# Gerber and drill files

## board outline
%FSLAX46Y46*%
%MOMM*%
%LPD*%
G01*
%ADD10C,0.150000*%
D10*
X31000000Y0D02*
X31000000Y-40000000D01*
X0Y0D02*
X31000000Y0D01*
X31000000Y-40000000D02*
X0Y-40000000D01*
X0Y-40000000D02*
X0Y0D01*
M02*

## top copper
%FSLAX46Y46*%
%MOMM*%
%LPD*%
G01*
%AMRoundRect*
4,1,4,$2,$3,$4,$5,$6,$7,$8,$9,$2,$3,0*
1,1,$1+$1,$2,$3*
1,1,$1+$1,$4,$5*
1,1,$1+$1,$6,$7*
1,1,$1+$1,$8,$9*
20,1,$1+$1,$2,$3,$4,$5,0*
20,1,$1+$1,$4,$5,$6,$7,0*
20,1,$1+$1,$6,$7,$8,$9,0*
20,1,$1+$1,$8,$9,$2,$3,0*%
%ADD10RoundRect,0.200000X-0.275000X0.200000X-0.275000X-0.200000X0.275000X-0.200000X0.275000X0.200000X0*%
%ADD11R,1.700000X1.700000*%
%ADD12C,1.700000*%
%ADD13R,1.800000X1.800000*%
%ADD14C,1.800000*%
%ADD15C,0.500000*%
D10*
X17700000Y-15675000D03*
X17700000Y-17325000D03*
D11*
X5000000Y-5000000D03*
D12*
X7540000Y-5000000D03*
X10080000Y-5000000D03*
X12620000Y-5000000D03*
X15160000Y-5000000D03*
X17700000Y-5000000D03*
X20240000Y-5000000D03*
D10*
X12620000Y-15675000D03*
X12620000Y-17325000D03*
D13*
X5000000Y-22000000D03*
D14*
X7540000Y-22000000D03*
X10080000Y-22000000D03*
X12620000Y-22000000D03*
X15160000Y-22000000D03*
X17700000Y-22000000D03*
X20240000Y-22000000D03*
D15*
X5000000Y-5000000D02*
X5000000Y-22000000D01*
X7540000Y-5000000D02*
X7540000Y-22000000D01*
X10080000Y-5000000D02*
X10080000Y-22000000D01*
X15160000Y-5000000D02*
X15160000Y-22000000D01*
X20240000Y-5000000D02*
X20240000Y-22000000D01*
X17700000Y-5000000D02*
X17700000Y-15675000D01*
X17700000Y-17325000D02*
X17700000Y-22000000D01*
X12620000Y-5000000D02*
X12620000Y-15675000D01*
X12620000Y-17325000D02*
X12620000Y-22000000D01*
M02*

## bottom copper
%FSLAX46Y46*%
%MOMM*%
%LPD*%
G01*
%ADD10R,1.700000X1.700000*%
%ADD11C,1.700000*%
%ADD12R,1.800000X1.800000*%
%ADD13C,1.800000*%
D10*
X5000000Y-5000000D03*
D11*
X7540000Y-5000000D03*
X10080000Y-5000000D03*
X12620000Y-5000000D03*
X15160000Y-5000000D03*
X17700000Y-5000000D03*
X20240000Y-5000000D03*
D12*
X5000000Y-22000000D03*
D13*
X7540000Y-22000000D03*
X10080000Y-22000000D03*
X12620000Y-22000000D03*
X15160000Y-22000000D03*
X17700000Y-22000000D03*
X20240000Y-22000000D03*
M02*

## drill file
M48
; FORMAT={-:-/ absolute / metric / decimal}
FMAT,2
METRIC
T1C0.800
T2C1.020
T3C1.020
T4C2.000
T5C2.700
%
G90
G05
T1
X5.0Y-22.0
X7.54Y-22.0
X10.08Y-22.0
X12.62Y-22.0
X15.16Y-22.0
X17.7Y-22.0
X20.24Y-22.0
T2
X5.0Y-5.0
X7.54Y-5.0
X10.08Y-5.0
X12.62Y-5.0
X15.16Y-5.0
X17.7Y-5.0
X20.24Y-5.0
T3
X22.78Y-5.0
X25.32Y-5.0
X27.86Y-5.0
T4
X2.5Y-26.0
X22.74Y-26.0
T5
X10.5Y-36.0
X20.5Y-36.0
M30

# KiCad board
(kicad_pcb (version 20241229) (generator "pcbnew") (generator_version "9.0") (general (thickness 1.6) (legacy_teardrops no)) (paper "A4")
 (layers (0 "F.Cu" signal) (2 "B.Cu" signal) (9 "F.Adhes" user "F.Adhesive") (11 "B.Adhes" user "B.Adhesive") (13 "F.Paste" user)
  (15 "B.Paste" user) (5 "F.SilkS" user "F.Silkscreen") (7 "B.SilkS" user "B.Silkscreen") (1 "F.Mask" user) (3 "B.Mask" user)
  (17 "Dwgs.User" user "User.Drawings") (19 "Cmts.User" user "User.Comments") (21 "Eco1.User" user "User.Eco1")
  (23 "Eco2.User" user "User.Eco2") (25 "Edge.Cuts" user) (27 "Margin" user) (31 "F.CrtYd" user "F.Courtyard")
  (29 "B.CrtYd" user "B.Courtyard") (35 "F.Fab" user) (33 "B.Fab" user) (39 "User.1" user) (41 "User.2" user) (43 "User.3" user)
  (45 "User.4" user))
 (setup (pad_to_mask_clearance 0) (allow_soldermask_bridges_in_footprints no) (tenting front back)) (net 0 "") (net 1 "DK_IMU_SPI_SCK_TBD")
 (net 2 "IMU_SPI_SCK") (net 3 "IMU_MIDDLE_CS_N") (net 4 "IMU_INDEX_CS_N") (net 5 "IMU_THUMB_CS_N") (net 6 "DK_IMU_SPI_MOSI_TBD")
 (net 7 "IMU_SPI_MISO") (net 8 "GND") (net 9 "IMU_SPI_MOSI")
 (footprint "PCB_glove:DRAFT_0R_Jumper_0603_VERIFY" (layer "F.Cu") (at 17.7 16.5 -90)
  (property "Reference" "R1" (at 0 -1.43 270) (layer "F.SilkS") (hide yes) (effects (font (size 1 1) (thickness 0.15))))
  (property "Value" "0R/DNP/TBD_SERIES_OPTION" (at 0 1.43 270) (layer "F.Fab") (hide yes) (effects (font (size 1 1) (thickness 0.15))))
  (pad "1" smd roundrect (at -0.825 0 270) (size 0.8 0.95) (layers "F.Cu" "F.Mask" "F.Paste") (roundrect_rratio 0.25)
   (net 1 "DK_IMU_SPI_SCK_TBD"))
  (pad "2" smd roundrect (at 0.825 0 270) (size 0.8 0.95) (layers "F.Cu" "F.Mask" "F.Paste") (roundrect_rratio 0.25) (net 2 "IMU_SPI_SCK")))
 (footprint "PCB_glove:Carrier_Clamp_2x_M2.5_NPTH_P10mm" (layer "F.Cu") (at 15.5 36)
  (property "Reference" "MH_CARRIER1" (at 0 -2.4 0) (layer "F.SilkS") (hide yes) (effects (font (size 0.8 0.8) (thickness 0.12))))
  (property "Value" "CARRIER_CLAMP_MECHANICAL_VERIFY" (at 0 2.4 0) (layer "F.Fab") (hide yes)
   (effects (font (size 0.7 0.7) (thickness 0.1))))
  (pad "" np_thru_hole circle (at -5 0) (size 2.7 2.7) (drill 2.7) (layers "*.Cu" "*.Mask"))
  (pad "" np_thru_hole circle (at 5 0) (size 2.7 2.7) (drill 2.7) (layers "*.Cu" "*.Mask")))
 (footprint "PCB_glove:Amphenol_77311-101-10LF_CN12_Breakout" (layer "F.Cu") (at 5 5)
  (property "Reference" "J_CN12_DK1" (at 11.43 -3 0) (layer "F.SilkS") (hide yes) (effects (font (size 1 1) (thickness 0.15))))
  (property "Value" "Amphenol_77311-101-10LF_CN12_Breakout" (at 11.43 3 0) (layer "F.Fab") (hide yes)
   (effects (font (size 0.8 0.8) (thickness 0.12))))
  (pad "" np_thru_hole circle (at 17.78 0) (size 1.02 1.02) (drill 1.02) (layers "*.Cu" "*.Mask"))
  (pad "" np_thru_hole circle (at 20.32 0) (size 1.02 1.02) (drill 1.02) (layers "*.Cu" "*.Mask"))
  (pad "" np_thru_hole circle (at 22.86 0) (size 1.02 1.02) (drill 1.02) (layers "*.Cu" "*.Mask"))
  (pad "1" thru_hole rect (at 0 0) (size 1.7 1.7) (drill 1.02) (layers "*.Cu" "*.Mask") (remove_unused_layers no) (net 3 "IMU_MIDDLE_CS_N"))
  (pad "2" thru_hole circle (at 2.54 0) (size 1.7 1.7) (drill 1.02) (layers "*.Cu" "*.Mask") (remove_unused_layers no)
   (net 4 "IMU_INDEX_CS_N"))
  (pad "3" thru_hole circle (at 5.08 0) (size 1.7 1.7) (drill 1.02) (layers "*.Cu" "*.Mask") (remove_unused_layers no)
   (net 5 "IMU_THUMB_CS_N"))
  (pad "4" thru_hole circle (at 7.62 0) (size 1.7 1.7) (drill 1.02) (layers "*.Cu" "*.Mask") (remove_unused_layers no)
   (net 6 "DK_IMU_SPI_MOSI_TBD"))
  (pad "5" thru_hole circle (at 10.16 0) (size 1.7 1.7) (drill 1.02) (layers "*.Cu" "*.Mask") (remove_unused_layers no)
   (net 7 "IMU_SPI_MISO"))
  (pad "6" thru_hole circle (at 12.7 0) (size 1.7 1.7) (drill 1.02) (layers "*.Cu" "*.Mask") (remove_unused_layers no)
   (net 1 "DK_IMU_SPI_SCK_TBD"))
  (pad "7" thru_hole circle (at 15.24 0) (size 1.7 1.7) (drill 1.02) (layers "*.Cu" "*.Mask") (remove_unused_layers no) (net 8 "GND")))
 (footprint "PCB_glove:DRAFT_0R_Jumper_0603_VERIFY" (layer "F.Cu") (at 12.62 16.5 -90)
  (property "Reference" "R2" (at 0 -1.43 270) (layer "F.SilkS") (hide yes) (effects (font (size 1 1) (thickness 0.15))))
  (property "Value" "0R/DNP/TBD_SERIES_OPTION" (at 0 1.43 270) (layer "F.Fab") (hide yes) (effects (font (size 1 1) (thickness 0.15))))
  (pad "1" smd roundrect (at -0.825 0 270) (size 0.8 0.95) (layers "F.Cu" "F.Mask" "F.Paste") (roundrect_rratio 0.25)
   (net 6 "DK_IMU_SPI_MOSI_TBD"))
  (pad "2" smd roundrect (at 0.825 0 270) (size 0.8 0.95) (layers "F.Cu" "F.Mask" "F.Paste") (roundrect_rratio 0.25) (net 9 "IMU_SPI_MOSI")))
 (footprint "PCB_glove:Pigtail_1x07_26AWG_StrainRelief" (layer "F.Cu") (at 5 22)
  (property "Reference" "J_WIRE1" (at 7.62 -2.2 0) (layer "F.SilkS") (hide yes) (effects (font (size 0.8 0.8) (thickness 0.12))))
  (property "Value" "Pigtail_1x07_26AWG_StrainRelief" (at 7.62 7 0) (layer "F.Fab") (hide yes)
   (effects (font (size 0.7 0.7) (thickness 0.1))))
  (pad "" np_thru_hole circle (at -2.5 4) (size 2 2) (drill 2) (layers "*.Cu" "*.Mask"))
  (pad "" np_thru_hole circle (at 17.74 4) (size 2 2) (drill 2) (layers "*.Cu" "*.Mask"))
  (pad "1" thru_hole rect (at 0 0) (size 1.8 1.8) (drill 0.8) (layers "*.Cu" "*.Mask") (remove_unused_layers no) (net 3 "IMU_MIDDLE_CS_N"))
  (pad "2" thru_hole circle (at 2.54 0) (size 1.8 1.8) (drill 0.8) (layers "*.Cu" "*.Mask") (remove_unused_layers no)
   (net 4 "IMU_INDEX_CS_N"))
  (pad "3" thru_hole circle (at 5.08 0) (size 1.8 1.8) (drill 0.8) (layers "*.Cu" "*.Mask") (remove_unused_layers no)
   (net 5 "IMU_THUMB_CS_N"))
  (pad "4" thru_hole circle (at 7.62 0) (size 1.8 1.8) (drill 0.8) (layers "*.Cu" "*.Mask") (remove_unused_layers no) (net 9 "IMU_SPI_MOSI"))
  (pad "5" thru_hole circle (at 10.16 0) (size 1.8 1.8) (drill 0.8) (layers "*.Cu" "*.Mask") (remove_unused_layers no)
   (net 7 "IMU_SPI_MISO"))
  (pad "6" thru_hole circle (at 12.7 0) (size 1.8 1.8) (drill 0.8) (layers "*.Cu" "*.Mask") (remove_unused_layers no) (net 2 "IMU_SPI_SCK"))
  (pad "7" thru_hole circle (at 15.24 0) (size 1.8 1.8) (drill 0.8) (layers "*.Cu" "*.Mask") (remove_unused_layers no) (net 8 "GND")))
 (gr_line (start 31 0) (end 31 40) (stroke (width 0.15) (type default)) (layer "Edge.Cuts"))
 (gr_line (start 0 0) (end 31 0) (stroke (width 0.15) (type default)) (layer "Edge.Cuts"))
 (gr_line (start 31 40) (end 0 40) (stroke (width 0.15) (type default)) (layer "Edge.Cuts"))
 (gr_line (start 0 40) (end 0 0) (stroke (width 0.15) (type default)) (layer "Edge.Cuts"))
 (segment (start 5 5) (end 5 22) (width 0.5) (layer "F.Cu") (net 3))
 (segment (start 7.54 5) (end 7.54 22) (width 0.5) (layer "F.Cu") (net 4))
 (segment (start 10.08 5) (end 10.08 22) (width 0.5) (layer "F.Cu") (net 5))
 (segment (start 15.16 5) (end 15.16 22) (width 0.5) (layer "F.Cu") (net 7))
 (segment (start 20.24 5) (end 20.24 22) (width 0.5) (layer "F.Cu") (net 8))
 (segment (start 17.7 5) (end 17.7 15.675) (width 0.5) (layer "F.Cu") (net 1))
 (segment (start 17.7 17.325) (end 17.7 22) (width 0.5) (layer "F.Cu") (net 2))
 (segment (start 12.62 5) (end 12.62 15.675) (width 0.5) (layer "F.Cu") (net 6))
 (segment (start 12.62 17.325) (end 12.62 22) (width 0.5) (layer "F.Cu") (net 9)))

